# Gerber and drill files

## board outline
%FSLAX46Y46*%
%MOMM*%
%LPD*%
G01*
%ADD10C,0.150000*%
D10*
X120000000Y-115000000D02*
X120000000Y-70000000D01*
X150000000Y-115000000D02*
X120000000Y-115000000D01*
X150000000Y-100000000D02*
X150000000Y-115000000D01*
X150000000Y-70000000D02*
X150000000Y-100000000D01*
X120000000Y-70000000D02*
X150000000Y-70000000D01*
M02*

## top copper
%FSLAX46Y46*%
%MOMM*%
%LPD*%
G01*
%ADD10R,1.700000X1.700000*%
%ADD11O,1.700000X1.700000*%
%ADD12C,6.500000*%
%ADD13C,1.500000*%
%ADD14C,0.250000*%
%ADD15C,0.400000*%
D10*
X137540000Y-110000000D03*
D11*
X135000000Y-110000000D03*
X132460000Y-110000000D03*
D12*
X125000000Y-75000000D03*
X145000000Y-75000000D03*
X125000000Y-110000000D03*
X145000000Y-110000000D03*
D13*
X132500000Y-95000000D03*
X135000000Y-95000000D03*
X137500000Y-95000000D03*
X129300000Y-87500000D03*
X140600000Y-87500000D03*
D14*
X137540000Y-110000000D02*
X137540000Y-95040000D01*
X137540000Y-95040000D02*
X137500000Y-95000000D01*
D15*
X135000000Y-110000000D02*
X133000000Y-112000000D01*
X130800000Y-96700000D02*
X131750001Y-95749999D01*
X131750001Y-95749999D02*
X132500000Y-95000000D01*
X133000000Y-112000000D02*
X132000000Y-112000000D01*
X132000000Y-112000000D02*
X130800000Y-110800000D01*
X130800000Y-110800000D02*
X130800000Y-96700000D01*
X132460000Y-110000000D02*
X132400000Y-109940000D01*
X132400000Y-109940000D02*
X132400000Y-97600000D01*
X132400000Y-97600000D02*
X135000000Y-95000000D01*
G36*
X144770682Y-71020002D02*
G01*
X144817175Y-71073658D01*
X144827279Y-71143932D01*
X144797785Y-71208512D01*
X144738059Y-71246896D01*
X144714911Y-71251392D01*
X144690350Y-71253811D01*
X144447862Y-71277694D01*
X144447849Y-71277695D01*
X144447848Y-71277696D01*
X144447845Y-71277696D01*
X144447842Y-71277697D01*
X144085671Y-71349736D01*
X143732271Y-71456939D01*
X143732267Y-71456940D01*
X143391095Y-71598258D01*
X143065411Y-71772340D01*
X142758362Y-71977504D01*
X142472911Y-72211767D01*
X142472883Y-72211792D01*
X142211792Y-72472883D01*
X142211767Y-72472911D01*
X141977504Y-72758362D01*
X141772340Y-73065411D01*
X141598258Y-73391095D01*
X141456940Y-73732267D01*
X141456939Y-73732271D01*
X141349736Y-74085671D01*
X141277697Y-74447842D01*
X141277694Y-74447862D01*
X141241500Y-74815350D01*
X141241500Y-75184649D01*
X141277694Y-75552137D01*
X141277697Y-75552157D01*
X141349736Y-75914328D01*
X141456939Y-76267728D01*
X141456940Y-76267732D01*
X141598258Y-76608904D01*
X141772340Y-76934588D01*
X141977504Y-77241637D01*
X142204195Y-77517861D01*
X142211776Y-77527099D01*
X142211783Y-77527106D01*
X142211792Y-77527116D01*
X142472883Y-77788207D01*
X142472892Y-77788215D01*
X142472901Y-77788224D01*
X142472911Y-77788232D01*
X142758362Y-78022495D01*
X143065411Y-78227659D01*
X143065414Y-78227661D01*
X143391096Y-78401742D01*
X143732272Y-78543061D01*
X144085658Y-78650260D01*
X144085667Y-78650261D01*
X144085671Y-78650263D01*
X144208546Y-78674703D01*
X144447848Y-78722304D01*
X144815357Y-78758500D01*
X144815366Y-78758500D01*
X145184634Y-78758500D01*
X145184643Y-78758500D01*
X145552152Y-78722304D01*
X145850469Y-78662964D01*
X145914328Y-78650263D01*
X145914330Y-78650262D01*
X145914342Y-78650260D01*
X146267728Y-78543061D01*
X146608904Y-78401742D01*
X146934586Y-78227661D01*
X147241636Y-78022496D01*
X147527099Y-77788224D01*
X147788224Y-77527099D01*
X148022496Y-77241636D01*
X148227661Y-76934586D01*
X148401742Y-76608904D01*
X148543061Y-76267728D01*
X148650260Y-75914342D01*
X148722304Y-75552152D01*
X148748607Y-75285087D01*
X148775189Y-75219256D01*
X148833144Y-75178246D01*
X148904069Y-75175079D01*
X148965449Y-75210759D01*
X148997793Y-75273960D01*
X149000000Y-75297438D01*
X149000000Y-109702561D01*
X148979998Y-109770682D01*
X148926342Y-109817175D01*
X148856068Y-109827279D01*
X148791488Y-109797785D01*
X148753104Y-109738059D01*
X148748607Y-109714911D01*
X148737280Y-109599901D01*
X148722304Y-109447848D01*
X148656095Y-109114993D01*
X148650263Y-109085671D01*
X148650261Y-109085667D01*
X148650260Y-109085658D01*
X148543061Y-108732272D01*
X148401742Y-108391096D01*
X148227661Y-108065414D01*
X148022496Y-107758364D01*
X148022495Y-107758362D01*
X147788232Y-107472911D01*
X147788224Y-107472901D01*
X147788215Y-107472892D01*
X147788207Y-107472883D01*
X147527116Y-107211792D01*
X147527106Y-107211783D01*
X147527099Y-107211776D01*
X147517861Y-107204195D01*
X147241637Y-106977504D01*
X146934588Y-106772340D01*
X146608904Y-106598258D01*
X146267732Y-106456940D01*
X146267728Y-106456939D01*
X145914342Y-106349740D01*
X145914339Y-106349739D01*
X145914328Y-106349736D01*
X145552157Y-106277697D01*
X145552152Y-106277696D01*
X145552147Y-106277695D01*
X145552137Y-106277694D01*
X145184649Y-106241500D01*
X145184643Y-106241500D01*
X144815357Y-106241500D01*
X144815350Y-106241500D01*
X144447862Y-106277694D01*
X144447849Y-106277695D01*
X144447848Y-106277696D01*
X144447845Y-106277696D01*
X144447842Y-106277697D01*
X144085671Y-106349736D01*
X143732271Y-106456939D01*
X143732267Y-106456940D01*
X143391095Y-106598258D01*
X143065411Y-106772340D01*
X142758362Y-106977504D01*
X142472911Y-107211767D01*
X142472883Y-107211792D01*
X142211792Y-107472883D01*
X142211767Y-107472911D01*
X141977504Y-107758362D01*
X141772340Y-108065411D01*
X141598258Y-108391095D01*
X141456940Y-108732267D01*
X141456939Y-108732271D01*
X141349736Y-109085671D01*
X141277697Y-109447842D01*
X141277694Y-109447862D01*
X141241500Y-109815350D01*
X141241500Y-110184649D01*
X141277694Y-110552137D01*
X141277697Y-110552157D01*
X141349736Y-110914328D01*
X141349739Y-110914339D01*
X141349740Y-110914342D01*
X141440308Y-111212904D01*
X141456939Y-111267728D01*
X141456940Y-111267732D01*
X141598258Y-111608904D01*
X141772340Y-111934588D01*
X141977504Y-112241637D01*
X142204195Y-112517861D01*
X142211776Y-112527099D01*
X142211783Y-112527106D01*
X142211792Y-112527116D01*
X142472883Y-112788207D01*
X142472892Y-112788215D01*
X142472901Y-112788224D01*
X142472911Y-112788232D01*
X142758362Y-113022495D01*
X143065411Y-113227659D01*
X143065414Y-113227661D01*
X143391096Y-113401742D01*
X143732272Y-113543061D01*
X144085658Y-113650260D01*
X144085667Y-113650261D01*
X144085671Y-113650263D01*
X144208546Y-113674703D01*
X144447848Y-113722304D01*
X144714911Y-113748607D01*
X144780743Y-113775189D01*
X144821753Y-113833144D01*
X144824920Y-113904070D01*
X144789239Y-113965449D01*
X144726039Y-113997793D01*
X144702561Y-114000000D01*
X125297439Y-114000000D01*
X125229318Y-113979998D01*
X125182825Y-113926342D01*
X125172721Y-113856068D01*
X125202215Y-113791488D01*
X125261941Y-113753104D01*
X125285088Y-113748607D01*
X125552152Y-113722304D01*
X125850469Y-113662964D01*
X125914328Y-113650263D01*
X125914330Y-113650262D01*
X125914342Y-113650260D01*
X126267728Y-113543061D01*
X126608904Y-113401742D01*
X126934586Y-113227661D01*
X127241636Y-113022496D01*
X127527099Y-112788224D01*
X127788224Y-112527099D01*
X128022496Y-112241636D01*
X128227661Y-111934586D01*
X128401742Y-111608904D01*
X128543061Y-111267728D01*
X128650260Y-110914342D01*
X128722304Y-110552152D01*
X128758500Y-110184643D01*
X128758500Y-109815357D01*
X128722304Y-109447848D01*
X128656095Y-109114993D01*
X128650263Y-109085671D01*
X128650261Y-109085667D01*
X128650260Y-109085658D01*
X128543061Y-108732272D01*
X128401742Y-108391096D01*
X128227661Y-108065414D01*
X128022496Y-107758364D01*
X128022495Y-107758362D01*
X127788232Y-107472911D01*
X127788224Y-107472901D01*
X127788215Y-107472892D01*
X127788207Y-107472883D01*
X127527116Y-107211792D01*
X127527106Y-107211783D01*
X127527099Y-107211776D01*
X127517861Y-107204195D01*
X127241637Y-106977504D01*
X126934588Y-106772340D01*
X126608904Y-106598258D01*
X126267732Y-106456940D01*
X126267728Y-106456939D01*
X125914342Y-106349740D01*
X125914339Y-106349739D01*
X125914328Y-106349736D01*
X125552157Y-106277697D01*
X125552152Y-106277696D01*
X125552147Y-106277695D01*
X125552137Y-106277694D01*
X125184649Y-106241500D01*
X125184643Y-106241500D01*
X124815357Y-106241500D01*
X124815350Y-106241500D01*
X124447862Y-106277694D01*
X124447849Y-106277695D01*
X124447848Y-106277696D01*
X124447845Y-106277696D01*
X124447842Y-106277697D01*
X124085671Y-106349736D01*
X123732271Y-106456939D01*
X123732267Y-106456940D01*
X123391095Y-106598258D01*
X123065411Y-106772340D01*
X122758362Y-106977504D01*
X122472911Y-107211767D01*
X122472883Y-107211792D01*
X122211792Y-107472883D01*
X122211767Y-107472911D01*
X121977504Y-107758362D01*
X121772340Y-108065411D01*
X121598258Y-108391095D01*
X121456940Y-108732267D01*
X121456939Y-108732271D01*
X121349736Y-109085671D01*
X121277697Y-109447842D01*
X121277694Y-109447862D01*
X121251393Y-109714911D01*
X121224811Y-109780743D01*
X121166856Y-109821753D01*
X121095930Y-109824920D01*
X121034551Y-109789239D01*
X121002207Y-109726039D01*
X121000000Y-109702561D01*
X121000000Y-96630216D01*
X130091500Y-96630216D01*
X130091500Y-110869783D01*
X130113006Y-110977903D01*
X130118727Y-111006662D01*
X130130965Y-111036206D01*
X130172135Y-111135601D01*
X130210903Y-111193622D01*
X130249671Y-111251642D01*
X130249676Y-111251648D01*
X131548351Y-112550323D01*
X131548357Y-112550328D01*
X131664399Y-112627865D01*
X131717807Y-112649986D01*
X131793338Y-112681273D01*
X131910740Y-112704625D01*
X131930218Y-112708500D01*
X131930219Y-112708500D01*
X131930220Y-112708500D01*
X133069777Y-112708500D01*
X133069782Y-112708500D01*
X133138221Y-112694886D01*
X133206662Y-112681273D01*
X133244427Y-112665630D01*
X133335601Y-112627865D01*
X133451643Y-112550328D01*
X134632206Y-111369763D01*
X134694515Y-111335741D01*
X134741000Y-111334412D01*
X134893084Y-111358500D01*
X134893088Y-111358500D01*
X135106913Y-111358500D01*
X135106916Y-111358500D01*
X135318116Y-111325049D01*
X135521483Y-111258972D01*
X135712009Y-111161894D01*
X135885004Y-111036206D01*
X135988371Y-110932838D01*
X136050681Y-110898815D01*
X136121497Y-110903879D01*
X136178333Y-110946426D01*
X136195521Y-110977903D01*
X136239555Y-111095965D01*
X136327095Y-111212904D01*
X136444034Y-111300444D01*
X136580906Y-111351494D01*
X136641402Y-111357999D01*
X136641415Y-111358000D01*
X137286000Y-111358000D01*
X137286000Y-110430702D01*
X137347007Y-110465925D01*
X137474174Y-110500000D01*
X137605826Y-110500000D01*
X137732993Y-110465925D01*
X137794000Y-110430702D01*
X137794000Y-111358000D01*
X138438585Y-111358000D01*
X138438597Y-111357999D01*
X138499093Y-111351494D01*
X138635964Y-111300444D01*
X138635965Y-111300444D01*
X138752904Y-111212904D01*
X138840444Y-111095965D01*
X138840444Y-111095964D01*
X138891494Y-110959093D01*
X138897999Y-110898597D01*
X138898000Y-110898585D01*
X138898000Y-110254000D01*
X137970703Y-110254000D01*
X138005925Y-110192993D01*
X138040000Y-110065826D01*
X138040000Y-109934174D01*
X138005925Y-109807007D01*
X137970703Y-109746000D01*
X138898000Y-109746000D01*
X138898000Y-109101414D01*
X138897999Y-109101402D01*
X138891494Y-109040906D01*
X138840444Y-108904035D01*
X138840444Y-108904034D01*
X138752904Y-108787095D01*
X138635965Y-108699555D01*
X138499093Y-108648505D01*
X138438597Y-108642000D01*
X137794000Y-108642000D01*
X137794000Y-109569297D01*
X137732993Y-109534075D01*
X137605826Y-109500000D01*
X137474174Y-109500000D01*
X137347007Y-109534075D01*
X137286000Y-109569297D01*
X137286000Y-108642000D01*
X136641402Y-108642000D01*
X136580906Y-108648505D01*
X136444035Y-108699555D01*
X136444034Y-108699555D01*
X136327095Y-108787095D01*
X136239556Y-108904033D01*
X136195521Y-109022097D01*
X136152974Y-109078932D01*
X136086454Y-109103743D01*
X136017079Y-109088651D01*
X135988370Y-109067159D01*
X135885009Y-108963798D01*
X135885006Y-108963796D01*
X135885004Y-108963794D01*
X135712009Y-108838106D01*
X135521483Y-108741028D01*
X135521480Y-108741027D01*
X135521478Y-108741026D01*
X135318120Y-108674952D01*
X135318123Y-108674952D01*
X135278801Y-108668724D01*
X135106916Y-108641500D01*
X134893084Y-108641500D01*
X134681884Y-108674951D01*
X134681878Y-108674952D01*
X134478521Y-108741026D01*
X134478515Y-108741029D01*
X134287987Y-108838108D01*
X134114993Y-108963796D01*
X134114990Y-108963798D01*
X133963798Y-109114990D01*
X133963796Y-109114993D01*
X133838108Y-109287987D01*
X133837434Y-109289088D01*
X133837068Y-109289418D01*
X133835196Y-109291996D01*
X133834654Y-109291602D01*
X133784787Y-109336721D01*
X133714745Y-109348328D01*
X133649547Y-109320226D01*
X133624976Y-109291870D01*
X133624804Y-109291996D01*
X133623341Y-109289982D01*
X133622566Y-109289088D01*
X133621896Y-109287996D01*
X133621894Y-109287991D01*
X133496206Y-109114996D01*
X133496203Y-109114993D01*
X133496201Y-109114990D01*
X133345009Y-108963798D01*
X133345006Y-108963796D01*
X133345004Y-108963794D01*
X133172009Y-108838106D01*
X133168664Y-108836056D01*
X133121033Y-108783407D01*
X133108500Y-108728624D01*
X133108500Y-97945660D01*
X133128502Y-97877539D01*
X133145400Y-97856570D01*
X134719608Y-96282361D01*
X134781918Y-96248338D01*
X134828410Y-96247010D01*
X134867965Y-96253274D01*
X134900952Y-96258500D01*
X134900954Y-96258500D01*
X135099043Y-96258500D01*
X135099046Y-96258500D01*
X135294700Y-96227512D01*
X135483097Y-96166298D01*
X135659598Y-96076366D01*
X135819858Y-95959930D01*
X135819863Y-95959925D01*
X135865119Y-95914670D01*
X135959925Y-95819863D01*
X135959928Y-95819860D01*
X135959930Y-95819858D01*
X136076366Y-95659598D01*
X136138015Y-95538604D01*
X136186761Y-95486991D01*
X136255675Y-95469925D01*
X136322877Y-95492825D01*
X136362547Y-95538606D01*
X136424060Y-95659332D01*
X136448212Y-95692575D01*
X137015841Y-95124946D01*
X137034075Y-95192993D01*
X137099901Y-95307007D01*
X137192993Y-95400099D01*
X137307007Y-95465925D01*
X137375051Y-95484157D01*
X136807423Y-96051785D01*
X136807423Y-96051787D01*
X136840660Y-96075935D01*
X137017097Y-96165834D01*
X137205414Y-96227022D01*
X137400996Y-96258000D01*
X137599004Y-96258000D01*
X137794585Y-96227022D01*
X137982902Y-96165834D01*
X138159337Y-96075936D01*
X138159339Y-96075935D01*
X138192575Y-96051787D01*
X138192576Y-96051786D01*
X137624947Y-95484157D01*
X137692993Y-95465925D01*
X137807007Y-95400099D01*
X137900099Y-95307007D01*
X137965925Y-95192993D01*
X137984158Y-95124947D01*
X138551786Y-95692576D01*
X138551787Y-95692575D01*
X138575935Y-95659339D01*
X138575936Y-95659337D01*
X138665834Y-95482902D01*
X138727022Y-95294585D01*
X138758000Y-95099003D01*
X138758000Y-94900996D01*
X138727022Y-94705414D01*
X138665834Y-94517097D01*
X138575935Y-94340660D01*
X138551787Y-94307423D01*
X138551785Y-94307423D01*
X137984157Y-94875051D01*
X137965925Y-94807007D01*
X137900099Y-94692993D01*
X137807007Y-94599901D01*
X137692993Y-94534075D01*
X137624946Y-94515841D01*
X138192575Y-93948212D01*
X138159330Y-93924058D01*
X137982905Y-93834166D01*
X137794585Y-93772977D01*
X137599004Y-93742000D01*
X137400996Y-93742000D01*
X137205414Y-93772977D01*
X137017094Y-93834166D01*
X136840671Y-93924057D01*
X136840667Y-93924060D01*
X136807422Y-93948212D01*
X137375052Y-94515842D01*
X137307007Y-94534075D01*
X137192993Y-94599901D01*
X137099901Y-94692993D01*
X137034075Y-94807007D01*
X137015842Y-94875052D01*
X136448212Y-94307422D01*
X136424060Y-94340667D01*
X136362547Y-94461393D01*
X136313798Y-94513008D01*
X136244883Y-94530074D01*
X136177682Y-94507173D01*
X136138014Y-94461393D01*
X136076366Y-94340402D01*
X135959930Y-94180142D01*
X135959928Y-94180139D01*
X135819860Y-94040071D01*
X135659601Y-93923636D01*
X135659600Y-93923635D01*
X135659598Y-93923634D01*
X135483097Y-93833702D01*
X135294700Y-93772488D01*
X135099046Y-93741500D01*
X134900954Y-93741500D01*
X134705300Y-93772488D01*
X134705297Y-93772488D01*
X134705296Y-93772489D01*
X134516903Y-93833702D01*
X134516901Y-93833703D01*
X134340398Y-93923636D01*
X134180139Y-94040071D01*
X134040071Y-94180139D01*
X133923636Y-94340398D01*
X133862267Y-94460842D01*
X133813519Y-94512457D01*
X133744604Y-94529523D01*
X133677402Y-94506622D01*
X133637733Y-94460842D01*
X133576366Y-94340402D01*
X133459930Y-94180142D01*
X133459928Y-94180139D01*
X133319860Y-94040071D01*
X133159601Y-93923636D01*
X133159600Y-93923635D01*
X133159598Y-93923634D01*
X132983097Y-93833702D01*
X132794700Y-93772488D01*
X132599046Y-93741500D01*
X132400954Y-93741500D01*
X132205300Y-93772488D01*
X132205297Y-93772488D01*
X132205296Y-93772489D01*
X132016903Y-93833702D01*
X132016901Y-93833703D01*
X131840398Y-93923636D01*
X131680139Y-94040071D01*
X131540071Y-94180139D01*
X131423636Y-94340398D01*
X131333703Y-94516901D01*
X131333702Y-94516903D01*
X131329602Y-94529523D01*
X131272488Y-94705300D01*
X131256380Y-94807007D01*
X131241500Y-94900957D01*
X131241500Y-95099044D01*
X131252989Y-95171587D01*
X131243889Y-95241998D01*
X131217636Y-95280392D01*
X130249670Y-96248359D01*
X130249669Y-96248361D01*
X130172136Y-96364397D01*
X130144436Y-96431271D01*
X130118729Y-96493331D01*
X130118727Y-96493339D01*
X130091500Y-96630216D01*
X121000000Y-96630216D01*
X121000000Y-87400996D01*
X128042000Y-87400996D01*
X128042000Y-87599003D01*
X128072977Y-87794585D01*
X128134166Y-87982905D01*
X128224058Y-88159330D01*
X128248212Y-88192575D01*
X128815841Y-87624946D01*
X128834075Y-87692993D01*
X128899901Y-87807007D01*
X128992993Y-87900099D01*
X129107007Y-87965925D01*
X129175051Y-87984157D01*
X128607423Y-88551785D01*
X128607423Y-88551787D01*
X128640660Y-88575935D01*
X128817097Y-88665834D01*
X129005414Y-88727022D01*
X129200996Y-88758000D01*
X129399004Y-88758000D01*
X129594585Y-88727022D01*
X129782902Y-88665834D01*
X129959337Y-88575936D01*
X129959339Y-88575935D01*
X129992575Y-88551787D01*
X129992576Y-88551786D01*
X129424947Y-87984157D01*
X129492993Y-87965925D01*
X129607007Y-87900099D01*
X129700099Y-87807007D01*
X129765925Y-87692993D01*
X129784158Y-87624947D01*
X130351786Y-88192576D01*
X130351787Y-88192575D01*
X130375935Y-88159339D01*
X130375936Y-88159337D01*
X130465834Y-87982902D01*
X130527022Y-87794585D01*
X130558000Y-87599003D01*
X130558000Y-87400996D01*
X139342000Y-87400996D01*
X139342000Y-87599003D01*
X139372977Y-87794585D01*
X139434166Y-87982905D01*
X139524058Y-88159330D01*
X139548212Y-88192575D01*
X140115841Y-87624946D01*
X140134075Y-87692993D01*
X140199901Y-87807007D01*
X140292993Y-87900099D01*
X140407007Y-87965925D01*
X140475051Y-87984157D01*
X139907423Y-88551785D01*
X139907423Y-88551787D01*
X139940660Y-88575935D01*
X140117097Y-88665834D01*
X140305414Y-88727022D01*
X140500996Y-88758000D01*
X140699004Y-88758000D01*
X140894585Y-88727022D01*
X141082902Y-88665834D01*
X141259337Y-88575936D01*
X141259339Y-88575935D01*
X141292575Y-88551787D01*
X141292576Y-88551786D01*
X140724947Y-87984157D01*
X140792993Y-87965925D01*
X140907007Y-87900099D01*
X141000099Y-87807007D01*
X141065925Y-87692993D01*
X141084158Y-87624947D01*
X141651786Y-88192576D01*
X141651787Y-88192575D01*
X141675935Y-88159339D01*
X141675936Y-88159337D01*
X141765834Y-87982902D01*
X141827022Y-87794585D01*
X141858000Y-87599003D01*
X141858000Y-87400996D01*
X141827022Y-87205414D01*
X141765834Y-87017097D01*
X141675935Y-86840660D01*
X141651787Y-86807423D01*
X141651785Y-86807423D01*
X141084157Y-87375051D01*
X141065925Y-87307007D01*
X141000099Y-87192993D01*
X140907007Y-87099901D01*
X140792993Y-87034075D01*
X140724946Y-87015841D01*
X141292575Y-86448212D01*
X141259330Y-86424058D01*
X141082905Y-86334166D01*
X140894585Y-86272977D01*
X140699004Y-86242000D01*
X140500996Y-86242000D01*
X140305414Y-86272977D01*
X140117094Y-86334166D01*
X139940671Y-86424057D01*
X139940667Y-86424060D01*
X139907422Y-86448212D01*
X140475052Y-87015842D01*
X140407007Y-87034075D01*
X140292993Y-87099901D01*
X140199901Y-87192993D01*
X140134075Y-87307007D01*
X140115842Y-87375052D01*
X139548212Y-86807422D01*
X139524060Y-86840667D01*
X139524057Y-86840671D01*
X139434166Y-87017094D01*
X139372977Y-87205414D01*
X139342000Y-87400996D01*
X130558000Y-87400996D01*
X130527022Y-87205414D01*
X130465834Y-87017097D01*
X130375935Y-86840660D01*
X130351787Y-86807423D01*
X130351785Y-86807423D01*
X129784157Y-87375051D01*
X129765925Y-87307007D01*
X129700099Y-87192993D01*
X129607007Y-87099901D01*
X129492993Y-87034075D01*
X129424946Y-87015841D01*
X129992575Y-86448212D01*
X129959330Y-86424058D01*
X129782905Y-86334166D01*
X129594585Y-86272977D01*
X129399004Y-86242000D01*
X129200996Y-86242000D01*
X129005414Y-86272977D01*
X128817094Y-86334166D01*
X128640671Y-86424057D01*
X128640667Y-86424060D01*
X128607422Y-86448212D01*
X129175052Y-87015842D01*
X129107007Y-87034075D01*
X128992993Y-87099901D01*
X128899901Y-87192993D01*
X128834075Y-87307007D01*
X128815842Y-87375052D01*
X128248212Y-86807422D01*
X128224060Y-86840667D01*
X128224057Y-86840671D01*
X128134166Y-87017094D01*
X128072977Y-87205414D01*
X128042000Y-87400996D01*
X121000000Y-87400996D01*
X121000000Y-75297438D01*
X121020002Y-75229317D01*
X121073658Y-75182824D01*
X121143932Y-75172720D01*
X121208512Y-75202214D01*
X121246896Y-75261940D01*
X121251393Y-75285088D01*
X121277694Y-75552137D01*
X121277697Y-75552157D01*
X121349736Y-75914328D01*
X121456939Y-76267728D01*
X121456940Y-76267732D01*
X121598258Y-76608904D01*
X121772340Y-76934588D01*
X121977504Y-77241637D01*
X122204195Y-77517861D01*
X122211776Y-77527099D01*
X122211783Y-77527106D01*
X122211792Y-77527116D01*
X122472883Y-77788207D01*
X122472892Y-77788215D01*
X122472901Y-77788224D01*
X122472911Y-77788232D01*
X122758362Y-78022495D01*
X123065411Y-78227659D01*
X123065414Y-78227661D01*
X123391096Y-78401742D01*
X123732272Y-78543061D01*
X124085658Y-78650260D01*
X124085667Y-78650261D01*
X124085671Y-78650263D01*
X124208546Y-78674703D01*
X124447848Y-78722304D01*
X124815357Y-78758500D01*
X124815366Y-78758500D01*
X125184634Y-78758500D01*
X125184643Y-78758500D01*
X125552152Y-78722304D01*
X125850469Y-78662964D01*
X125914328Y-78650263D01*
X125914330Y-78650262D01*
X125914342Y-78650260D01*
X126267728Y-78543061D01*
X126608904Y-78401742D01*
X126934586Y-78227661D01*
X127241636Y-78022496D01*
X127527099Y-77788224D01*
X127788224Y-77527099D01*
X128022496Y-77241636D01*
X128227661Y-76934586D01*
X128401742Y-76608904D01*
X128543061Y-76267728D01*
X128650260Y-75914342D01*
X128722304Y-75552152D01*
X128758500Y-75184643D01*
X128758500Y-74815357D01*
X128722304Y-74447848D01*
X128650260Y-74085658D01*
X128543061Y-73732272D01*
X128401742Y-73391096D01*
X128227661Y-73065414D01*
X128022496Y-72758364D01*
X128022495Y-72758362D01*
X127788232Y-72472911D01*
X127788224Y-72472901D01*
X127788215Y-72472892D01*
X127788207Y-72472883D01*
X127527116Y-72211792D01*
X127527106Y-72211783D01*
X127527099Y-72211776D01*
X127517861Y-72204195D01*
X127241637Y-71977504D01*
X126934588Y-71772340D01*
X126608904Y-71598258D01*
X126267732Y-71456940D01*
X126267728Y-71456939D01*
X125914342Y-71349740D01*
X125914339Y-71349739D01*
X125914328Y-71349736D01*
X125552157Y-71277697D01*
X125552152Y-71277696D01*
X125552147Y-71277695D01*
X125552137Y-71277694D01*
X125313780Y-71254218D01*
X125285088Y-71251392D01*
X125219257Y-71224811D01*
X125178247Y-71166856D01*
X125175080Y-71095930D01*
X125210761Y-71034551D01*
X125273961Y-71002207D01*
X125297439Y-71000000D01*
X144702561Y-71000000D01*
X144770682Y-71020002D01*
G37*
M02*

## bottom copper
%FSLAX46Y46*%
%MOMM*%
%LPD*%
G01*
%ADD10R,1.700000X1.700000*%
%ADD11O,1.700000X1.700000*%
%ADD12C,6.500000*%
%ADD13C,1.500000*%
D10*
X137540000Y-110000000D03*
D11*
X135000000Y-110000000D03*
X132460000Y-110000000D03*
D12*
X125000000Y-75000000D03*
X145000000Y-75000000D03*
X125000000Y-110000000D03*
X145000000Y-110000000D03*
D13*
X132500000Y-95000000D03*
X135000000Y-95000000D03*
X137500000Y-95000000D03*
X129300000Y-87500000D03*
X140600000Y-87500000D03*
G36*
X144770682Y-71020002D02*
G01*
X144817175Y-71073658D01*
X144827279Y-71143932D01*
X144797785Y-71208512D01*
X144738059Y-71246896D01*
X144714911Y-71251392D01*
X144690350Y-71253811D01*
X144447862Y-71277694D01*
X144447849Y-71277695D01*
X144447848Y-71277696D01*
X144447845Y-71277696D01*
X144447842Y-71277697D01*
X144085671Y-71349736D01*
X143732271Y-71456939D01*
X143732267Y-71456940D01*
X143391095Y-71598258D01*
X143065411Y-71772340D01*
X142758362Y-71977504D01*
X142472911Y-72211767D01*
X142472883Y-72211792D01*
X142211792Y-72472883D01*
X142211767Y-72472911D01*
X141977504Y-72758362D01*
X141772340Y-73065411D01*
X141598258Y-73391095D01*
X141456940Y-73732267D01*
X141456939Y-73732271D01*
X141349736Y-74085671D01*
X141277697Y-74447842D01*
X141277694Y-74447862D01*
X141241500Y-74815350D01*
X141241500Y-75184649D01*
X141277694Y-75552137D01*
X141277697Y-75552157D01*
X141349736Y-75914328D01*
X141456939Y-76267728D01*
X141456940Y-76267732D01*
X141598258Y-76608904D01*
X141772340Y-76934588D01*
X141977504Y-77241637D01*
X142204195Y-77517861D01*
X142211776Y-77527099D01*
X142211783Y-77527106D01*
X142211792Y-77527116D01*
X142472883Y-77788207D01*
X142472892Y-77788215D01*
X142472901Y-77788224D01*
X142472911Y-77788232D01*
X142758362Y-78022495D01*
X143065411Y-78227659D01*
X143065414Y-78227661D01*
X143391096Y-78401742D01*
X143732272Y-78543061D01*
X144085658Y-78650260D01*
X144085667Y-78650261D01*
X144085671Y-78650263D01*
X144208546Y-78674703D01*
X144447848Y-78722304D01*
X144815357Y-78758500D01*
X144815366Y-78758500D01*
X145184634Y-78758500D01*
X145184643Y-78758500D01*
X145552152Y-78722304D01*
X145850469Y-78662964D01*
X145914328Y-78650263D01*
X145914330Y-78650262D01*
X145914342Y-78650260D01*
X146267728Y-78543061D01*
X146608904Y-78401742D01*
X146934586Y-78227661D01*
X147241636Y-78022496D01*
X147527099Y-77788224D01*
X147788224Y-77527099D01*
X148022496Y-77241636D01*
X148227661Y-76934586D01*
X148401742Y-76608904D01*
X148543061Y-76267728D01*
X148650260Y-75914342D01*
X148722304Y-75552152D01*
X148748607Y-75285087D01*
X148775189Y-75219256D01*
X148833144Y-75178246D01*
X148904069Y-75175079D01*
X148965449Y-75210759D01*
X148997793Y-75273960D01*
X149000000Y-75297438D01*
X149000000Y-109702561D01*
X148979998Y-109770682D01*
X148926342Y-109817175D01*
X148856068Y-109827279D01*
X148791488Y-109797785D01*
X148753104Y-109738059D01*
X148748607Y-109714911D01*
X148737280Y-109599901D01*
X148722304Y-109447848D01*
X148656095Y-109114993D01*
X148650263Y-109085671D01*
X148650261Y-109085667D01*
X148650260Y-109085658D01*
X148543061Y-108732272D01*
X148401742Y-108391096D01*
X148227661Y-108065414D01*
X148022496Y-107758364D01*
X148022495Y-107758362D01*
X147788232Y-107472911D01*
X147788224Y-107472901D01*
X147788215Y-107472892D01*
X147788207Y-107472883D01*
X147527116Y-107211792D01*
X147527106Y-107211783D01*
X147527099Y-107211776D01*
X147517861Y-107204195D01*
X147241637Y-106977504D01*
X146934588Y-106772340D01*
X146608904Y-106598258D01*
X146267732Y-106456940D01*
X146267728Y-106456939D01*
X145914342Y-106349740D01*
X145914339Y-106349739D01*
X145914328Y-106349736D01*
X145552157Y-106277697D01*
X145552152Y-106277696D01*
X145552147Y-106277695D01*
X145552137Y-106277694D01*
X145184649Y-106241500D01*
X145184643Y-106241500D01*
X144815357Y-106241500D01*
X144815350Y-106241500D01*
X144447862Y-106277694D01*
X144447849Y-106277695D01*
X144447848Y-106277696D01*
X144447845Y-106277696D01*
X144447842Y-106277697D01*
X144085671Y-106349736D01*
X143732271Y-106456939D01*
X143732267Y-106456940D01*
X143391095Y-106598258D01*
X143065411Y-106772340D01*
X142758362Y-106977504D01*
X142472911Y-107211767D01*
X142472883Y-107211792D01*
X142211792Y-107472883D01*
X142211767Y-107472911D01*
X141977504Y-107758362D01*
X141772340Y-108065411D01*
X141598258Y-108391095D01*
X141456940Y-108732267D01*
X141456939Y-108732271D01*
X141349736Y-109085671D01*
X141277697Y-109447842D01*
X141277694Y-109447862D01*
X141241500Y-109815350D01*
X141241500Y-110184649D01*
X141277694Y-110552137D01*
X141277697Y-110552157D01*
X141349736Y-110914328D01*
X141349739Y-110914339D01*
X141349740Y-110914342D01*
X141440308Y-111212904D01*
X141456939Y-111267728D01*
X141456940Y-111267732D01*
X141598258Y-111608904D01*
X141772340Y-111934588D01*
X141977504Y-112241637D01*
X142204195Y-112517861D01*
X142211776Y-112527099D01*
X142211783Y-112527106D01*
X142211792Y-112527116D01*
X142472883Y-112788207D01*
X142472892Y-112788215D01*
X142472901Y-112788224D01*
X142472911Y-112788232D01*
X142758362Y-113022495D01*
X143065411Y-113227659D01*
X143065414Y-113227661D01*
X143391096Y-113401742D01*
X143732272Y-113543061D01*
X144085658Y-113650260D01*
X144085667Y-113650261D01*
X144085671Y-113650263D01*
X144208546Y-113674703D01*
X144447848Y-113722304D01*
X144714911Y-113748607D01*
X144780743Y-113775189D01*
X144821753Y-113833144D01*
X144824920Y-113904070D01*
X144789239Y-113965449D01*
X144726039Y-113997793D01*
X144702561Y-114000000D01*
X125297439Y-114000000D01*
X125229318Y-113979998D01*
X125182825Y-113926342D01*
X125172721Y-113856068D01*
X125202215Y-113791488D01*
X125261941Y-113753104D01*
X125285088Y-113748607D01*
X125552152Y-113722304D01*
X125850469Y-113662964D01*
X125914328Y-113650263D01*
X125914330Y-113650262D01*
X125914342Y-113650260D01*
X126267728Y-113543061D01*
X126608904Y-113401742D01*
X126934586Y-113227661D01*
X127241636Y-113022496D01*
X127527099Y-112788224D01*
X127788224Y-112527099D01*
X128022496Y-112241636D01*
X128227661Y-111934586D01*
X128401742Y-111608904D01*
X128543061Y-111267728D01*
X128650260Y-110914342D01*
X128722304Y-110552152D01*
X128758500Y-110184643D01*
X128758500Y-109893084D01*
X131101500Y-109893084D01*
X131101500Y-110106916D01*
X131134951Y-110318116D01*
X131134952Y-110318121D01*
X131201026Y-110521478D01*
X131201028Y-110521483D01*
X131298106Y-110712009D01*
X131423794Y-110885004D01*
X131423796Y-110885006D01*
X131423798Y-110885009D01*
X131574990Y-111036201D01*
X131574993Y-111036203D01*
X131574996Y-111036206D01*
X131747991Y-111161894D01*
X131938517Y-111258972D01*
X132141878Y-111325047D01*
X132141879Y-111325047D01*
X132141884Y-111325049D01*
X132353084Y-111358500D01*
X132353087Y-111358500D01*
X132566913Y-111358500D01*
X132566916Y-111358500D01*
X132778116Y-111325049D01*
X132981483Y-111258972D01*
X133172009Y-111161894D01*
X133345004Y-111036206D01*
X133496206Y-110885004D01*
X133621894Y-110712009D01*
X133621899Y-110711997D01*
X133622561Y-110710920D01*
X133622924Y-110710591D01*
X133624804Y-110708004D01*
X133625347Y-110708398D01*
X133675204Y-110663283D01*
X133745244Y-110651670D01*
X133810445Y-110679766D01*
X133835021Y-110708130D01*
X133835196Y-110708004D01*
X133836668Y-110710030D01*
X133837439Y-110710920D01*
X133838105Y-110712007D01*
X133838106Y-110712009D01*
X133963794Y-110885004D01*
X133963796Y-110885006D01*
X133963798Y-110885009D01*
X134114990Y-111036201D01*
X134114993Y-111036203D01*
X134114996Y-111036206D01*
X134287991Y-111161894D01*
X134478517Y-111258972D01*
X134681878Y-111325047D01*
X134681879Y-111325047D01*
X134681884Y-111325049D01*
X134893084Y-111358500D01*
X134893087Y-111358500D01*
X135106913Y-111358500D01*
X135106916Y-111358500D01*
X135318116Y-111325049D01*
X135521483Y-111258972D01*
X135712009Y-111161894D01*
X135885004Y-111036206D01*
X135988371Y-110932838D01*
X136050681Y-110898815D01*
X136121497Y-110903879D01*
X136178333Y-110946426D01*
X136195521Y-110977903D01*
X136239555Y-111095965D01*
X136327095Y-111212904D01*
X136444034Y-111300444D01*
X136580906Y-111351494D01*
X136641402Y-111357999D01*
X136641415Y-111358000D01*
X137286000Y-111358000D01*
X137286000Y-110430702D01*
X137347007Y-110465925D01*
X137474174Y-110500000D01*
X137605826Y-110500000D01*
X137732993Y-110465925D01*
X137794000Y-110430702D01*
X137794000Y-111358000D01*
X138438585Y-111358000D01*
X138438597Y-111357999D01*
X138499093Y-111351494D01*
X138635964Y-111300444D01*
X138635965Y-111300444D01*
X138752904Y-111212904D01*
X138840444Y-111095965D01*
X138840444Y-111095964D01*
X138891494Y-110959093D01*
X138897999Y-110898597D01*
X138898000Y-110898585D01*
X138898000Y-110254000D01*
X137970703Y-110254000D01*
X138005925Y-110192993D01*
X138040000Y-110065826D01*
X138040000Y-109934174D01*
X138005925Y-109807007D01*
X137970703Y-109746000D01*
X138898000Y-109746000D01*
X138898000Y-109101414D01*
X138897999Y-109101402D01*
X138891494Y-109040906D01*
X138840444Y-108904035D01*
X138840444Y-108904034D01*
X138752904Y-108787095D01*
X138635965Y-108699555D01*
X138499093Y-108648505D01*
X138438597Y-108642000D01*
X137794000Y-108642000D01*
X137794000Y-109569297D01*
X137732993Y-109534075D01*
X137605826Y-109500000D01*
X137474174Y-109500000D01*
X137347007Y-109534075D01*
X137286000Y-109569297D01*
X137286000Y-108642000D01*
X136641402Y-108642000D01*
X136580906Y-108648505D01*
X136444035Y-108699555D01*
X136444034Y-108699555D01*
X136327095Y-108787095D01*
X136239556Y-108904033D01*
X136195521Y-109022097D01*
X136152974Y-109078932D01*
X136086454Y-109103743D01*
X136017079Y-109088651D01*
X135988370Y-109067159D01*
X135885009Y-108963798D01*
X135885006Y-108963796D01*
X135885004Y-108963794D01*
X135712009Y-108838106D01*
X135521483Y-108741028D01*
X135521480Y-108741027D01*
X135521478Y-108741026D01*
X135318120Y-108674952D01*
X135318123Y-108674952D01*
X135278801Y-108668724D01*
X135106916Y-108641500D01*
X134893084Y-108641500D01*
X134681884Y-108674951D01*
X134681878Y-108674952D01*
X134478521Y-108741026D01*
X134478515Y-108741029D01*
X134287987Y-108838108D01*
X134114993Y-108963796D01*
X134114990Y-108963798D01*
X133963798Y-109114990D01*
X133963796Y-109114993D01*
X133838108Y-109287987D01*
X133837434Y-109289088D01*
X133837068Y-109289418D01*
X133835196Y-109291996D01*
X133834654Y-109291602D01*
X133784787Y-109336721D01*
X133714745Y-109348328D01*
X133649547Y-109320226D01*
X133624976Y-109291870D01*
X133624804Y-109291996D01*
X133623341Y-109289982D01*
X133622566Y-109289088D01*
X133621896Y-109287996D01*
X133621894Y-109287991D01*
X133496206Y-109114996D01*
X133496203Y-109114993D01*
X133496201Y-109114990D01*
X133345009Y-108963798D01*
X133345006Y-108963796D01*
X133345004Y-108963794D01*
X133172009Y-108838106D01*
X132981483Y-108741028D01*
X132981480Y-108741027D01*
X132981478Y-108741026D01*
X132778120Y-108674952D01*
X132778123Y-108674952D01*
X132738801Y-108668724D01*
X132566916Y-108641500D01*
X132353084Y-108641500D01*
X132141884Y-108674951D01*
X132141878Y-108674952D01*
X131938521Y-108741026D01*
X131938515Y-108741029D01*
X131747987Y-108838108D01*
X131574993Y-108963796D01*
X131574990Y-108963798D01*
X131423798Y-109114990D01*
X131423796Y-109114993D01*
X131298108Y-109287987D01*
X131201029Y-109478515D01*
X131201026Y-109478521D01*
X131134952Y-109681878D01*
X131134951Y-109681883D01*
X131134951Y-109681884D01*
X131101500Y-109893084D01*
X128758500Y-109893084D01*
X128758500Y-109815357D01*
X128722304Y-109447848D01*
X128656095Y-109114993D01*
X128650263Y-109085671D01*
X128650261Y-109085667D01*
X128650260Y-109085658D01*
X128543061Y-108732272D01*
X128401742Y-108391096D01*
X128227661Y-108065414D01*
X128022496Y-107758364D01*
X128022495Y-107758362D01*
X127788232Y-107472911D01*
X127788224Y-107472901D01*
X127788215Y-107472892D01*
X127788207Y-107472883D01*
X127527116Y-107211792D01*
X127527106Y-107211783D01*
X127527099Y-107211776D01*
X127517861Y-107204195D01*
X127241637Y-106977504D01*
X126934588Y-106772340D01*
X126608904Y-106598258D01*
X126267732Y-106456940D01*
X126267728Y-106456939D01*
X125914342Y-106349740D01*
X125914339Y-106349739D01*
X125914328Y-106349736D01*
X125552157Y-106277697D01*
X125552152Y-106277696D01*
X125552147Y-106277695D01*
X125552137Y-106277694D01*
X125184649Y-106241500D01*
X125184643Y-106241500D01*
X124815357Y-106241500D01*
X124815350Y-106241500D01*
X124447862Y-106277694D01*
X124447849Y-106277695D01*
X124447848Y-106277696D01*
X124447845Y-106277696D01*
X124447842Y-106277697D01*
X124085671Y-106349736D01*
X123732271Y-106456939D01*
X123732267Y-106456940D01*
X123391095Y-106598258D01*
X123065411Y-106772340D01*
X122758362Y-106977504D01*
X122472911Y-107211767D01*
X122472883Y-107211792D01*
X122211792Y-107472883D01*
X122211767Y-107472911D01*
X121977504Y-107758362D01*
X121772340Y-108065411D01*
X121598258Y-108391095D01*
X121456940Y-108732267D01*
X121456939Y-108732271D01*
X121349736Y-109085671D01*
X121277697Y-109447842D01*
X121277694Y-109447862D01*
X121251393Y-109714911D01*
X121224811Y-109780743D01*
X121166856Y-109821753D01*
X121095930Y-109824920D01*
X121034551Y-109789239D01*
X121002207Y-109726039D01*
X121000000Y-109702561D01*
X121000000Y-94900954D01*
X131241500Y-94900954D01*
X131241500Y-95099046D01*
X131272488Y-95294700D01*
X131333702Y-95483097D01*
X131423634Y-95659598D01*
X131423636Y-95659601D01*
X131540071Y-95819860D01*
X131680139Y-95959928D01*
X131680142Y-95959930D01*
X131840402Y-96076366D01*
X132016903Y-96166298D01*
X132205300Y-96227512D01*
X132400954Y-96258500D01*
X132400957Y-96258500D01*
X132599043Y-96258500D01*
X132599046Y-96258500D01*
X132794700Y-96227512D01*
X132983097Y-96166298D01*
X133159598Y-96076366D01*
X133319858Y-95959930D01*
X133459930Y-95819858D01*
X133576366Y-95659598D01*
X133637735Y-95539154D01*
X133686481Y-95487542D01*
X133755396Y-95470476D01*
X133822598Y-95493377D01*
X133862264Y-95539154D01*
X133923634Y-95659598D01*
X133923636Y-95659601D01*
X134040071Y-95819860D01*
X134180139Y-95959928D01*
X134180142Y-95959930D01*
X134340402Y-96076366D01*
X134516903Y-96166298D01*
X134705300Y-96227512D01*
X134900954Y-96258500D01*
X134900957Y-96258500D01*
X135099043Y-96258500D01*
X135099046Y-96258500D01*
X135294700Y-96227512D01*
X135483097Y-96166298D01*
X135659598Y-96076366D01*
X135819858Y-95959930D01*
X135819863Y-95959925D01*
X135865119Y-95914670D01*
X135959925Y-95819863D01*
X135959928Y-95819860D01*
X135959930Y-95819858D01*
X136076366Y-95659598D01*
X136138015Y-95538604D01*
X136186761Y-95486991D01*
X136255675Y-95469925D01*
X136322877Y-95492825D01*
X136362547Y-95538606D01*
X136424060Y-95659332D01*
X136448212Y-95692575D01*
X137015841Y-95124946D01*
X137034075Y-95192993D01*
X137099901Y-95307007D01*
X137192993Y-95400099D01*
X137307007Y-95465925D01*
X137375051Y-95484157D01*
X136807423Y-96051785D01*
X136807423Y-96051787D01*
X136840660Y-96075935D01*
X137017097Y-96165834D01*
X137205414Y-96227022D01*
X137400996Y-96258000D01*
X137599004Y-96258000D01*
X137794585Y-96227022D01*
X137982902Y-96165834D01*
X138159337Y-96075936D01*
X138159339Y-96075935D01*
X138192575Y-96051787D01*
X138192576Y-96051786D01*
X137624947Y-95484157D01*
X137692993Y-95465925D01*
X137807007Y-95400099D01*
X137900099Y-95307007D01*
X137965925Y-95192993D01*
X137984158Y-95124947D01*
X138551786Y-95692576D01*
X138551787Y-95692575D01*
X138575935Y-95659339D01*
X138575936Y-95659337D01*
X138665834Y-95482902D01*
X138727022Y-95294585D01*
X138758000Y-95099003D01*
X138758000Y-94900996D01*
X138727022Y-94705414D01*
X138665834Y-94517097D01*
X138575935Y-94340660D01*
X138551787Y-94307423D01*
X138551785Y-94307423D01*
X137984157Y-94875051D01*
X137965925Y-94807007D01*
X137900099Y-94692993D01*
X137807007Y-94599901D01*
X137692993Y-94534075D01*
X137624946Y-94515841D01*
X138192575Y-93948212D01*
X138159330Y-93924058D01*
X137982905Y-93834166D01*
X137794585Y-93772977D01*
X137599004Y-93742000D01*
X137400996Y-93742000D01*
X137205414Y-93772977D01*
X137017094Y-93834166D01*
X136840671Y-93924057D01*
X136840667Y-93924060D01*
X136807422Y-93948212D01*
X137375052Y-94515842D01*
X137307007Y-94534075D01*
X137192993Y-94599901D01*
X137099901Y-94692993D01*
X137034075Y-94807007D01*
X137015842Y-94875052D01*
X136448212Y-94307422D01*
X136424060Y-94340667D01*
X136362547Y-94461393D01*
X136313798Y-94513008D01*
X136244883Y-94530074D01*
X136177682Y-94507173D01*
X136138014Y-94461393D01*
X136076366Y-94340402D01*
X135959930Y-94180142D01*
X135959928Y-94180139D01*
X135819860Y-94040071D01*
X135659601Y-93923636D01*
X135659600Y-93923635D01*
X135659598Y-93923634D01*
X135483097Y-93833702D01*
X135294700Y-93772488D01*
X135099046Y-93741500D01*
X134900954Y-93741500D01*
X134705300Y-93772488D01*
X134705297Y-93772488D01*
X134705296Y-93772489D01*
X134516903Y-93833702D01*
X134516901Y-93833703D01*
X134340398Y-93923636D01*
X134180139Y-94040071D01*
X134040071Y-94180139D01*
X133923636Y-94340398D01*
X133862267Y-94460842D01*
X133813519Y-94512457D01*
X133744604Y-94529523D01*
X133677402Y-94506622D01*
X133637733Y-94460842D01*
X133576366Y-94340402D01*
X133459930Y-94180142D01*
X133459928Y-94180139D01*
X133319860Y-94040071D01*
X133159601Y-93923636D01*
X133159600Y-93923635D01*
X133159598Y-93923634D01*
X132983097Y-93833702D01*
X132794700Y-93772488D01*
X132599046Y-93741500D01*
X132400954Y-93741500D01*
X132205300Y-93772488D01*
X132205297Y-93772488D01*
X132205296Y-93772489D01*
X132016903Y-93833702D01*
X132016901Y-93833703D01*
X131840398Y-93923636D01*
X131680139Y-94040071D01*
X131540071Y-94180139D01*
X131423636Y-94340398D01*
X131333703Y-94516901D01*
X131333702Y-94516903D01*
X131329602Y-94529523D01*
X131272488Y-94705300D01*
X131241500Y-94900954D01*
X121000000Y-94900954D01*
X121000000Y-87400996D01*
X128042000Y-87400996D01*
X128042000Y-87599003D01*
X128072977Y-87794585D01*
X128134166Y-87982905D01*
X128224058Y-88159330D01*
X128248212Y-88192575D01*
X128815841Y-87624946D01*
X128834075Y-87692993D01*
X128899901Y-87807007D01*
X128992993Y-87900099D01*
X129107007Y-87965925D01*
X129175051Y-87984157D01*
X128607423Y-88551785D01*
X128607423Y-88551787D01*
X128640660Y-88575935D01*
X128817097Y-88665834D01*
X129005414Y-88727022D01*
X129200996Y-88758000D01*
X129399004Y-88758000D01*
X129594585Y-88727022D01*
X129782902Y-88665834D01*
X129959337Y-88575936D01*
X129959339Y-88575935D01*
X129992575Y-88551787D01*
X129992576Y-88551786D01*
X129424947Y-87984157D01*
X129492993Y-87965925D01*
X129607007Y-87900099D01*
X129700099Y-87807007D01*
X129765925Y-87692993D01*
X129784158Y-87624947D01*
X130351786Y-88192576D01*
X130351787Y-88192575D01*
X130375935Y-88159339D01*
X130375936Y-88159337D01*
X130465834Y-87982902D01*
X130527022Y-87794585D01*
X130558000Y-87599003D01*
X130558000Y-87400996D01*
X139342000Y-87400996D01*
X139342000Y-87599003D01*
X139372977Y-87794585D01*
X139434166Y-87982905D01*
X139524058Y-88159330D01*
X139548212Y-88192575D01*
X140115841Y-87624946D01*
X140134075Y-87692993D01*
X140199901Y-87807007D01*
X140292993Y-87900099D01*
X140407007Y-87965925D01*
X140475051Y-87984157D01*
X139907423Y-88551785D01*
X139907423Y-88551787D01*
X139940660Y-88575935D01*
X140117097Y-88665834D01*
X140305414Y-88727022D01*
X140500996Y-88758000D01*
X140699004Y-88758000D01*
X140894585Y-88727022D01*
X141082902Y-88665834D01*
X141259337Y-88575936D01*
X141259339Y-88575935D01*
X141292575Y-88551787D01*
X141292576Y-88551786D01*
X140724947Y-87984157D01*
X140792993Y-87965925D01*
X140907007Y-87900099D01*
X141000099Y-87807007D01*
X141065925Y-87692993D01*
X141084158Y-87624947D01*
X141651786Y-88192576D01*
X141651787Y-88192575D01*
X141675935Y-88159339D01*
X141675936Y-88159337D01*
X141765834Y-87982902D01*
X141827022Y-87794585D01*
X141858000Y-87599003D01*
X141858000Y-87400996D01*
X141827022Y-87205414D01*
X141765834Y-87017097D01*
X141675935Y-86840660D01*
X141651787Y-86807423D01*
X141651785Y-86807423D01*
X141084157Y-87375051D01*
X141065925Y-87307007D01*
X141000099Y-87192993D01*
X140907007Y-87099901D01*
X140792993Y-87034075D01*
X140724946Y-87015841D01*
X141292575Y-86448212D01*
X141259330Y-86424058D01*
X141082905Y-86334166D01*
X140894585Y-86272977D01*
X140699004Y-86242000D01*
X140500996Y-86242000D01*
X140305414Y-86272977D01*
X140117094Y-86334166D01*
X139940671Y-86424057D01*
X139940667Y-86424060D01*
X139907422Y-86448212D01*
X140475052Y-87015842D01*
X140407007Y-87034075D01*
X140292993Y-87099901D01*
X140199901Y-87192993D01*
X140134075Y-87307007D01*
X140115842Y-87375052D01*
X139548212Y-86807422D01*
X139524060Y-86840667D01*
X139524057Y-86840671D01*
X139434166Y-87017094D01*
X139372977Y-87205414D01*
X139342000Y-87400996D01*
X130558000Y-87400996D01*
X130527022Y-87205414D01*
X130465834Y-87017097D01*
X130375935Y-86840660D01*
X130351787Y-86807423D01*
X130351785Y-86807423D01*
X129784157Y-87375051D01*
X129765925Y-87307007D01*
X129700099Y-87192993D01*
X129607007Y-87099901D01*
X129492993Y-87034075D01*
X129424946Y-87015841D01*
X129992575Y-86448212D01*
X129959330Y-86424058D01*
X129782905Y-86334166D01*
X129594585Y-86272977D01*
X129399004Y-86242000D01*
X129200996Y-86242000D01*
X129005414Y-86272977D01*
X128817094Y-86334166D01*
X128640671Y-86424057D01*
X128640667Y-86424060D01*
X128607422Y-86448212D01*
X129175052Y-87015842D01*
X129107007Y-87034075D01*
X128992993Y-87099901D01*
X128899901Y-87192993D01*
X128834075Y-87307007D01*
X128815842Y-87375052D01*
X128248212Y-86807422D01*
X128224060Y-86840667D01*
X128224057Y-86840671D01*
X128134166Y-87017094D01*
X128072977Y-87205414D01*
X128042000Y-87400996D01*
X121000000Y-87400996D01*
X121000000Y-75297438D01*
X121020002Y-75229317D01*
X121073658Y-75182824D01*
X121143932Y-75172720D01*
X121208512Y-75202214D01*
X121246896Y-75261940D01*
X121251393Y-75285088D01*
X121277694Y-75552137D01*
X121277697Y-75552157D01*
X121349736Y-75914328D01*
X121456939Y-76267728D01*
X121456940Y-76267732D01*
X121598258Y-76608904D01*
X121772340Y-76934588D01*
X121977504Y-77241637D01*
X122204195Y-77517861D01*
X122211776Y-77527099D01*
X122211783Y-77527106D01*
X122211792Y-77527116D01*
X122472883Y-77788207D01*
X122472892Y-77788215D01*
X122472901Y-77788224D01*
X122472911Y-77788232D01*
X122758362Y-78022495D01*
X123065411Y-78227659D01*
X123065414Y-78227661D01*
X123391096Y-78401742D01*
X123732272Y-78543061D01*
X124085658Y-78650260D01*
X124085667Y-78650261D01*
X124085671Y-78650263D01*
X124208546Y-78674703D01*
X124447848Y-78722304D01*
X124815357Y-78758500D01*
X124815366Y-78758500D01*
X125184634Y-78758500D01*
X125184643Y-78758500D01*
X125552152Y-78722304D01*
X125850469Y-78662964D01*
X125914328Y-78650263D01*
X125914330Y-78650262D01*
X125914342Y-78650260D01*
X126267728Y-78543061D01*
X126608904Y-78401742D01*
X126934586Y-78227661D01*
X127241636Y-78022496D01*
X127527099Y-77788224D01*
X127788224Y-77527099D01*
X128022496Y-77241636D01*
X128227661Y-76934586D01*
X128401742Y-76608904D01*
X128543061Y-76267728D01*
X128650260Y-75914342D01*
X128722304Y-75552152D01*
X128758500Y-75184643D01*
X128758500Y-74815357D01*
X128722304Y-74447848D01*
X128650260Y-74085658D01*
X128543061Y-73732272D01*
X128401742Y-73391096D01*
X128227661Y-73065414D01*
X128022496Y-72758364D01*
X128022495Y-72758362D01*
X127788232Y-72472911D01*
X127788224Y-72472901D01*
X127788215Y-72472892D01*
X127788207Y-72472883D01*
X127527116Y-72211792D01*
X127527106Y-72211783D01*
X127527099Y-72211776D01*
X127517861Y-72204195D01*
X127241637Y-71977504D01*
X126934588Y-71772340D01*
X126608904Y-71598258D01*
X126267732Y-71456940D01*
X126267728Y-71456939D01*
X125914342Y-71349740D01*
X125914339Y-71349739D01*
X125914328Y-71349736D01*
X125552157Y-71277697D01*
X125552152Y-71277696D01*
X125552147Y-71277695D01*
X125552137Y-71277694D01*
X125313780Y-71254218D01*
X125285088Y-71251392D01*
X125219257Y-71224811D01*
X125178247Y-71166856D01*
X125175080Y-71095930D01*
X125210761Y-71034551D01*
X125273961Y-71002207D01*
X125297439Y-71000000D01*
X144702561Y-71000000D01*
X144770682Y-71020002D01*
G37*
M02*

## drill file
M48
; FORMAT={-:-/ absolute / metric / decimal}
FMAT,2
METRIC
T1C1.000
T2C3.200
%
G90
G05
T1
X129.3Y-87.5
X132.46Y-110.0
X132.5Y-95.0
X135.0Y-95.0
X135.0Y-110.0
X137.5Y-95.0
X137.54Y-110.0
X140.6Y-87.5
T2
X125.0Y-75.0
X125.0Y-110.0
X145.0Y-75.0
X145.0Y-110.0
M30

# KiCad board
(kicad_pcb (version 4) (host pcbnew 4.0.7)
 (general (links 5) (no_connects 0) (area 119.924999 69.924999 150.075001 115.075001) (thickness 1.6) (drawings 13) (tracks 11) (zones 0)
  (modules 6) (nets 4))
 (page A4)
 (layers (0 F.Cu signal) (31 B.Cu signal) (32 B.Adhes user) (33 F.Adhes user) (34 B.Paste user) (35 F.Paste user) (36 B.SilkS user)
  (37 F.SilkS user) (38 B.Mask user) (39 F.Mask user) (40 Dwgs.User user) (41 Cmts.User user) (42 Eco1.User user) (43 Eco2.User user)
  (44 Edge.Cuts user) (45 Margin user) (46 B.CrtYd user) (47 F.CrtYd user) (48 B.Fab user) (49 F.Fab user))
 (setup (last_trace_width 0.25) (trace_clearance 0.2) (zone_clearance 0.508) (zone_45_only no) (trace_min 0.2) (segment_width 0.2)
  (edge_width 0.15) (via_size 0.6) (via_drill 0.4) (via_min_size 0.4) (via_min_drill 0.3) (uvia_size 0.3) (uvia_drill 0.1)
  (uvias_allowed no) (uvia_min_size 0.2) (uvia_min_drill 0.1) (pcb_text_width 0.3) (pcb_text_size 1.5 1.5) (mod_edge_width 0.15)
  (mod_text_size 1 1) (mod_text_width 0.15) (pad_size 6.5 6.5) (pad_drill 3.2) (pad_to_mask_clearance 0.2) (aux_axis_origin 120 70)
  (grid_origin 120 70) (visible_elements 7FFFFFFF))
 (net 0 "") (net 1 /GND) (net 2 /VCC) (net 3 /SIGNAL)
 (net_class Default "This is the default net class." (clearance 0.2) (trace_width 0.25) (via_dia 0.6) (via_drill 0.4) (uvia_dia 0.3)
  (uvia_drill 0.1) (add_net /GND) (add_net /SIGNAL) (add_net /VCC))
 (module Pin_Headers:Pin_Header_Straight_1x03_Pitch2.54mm (layer F.Cu) (at 137.54 110 270)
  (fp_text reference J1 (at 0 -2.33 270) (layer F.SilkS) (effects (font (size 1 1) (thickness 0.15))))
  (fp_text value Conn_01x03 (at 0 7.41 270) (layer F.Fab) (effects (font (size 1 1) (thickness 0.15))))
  (pad 1 thru_hole rect (at 0 0 270) (size 1.7 1.7) (drill 1) (layers *.Cu *.Mask) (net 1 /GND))
  (pad 2 thru_hole oval (at 0 2.54 270) (size 1.7 1.7) (drill 1) (layers *.Cu *.Mask) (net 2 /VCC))
  (pad 3 thru_hole oval (at 0 5.08 270) (size 1.7 1.7) (drill 1) (layers *.Cu *.Mask) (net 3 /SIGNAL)))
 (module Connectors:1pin (layer F.Cu) (at 125 75)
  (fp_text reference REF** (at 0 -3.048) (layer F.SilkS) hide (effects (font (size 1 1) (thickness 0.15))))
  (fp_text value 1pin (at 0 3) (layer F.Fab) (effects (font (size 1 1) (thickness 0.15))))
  (pad ~ thru_hole circle (at 0 0) (size 6.5 6.5) (drill 3.2) (layers *.Cu *.Mask)))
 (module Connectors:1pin (layer F.Cu) (at 145 75)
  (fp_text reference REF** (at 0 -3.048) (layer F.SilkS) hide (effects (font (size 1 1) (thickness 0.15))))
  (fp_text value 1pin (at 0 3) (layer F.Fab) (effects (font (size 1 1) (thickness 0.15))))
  (pad ~ thru_hole circle (at 0 0) (size 6.5 6.5) (drill 3.2) (layers *.Cu *.Mask)))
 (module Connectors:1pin (layer F.Cu) (at 125 110)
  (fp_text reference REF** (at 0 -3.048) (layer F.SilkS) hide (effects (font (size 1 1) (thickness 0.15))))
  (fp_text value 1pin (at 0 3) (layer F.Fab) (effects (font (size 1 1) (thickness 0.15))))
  (pad ~ thru_hole circle (at 0 0) (size 6.5 6.5) (drill 3.2) (layers *.Cu *.Mask)))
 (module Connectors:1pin (layer F.Cu) (at 145 110)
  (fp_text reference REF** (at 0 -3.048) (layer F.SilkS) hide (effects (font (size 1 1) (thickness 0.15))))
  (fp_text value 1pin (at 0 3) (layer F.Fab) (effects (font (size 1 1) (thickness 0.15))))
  (pad ~ thru_hole circle (at 0 0) (size 6.5 6.5) (drill 3.2) (layers *.Cu *.Mask)))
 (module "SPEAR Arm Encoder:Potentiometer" (layer F.Cu) (at 135 90)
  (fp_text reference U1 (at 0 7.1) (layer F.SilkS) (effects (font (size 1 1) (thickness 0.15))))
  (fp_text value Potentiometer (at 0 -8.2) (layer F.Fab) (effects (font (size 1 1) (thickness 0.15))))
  (pad 1 thru_hole circle (at -2.5 5) (size 1.5 1.5) (drill 1) (layers *.Cu *.Mask) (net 2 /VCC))
  (pad 2 thru_hole circle (at 0 5) (size 1.5 1.5) (drill 1) (layers *.Cu *.Mask) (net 3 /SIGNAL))
  (pad 3 thru_hole circle (at 2.5 5) (size 1.5 1.5) (drill 1) (layers *.Cu *.Mask) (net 1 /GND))
  (pad 4 thru_hole circle (at -5.7 -2.5) (size 1.5 1.5) (drill 1) (layers *.Cu *.Mask) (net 1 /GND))
  (pad 5 thru_hole circle (at 5.6 -2.5) (size 1.5 1.5) (drill 1) (layers *.Cu *.Mask) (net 1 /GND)))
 (gr_line (start 120 115) (end 120 70) (layer Edge.Cuts) (width 0.15))
 (gr_line (start 150 115) (end 120 115) (layer Edge.Cuts) (width 0.15))
 (gr_line (start 150 100) (end 150 115) (layer Edge.Cuts) (width 0.15))
 (gr_line (start 150 70) (end 150 100) (layer Edge.Cuts) (width 0.15))
 (gr_line (start 120 70) (end 150 70) (layer Edge.Cuts) (width 0.15))
 (segment (start 137.54 110) (end 137.54 95.04) (width 0.25) (layer F.Cu) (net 1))
 (segment (start 137.54 95.04) (end 137.5 95) (width 0.25) (layer F.Cu) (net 1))
 (segment (start 135 110) (end 133 112) (width 0.4) (layer F.Cu) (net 2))
 (segment (start 130.8 96.7) (end 131.750001 95.749999) (width 0.4) (layer F.Cu) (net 2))
 (segment (start 131.750001 95.749999) (end 132.5 95) (width 0.4) (layer F.Cu) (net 2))
 (segment (start 133 112) (end 132 112) (width 0.4) (layer F.Cu) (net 2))
 (segment (start 132 112) (end 130.8 110.8) (width 0.4) (layer F.Cu) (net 2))
 (segment (start 130.8 110.8) (end 130.8 96.7) (width 0.4) (layer F.Cu) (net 2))
 (segment (start 132.46 110) (end 132.4 109.94) (width 0.4) (layer F.Cu) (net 3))
 (segment (start 132.4 109.94) (end 132.4 97.6) (width 0.4) (layer F.Cu) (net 3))
 (segment (start 132.4 97.6) (end 135 95) (width 0.4) (layer F.Cu) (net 3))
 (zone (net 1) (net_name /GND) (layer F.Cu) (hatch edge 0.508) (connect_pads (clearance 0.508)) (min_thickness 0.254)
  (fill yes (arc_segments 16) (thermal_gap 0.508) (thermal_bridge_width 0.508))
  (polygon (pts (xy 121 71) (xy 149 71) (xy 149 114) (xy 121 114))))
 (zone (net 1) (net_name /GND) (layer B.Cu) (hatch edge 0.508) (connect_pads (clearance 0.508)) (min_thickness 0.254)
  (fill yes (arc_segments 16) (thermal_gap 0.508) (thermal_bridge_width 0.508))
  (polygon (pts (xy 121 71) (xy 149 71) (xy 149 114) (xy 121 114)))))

